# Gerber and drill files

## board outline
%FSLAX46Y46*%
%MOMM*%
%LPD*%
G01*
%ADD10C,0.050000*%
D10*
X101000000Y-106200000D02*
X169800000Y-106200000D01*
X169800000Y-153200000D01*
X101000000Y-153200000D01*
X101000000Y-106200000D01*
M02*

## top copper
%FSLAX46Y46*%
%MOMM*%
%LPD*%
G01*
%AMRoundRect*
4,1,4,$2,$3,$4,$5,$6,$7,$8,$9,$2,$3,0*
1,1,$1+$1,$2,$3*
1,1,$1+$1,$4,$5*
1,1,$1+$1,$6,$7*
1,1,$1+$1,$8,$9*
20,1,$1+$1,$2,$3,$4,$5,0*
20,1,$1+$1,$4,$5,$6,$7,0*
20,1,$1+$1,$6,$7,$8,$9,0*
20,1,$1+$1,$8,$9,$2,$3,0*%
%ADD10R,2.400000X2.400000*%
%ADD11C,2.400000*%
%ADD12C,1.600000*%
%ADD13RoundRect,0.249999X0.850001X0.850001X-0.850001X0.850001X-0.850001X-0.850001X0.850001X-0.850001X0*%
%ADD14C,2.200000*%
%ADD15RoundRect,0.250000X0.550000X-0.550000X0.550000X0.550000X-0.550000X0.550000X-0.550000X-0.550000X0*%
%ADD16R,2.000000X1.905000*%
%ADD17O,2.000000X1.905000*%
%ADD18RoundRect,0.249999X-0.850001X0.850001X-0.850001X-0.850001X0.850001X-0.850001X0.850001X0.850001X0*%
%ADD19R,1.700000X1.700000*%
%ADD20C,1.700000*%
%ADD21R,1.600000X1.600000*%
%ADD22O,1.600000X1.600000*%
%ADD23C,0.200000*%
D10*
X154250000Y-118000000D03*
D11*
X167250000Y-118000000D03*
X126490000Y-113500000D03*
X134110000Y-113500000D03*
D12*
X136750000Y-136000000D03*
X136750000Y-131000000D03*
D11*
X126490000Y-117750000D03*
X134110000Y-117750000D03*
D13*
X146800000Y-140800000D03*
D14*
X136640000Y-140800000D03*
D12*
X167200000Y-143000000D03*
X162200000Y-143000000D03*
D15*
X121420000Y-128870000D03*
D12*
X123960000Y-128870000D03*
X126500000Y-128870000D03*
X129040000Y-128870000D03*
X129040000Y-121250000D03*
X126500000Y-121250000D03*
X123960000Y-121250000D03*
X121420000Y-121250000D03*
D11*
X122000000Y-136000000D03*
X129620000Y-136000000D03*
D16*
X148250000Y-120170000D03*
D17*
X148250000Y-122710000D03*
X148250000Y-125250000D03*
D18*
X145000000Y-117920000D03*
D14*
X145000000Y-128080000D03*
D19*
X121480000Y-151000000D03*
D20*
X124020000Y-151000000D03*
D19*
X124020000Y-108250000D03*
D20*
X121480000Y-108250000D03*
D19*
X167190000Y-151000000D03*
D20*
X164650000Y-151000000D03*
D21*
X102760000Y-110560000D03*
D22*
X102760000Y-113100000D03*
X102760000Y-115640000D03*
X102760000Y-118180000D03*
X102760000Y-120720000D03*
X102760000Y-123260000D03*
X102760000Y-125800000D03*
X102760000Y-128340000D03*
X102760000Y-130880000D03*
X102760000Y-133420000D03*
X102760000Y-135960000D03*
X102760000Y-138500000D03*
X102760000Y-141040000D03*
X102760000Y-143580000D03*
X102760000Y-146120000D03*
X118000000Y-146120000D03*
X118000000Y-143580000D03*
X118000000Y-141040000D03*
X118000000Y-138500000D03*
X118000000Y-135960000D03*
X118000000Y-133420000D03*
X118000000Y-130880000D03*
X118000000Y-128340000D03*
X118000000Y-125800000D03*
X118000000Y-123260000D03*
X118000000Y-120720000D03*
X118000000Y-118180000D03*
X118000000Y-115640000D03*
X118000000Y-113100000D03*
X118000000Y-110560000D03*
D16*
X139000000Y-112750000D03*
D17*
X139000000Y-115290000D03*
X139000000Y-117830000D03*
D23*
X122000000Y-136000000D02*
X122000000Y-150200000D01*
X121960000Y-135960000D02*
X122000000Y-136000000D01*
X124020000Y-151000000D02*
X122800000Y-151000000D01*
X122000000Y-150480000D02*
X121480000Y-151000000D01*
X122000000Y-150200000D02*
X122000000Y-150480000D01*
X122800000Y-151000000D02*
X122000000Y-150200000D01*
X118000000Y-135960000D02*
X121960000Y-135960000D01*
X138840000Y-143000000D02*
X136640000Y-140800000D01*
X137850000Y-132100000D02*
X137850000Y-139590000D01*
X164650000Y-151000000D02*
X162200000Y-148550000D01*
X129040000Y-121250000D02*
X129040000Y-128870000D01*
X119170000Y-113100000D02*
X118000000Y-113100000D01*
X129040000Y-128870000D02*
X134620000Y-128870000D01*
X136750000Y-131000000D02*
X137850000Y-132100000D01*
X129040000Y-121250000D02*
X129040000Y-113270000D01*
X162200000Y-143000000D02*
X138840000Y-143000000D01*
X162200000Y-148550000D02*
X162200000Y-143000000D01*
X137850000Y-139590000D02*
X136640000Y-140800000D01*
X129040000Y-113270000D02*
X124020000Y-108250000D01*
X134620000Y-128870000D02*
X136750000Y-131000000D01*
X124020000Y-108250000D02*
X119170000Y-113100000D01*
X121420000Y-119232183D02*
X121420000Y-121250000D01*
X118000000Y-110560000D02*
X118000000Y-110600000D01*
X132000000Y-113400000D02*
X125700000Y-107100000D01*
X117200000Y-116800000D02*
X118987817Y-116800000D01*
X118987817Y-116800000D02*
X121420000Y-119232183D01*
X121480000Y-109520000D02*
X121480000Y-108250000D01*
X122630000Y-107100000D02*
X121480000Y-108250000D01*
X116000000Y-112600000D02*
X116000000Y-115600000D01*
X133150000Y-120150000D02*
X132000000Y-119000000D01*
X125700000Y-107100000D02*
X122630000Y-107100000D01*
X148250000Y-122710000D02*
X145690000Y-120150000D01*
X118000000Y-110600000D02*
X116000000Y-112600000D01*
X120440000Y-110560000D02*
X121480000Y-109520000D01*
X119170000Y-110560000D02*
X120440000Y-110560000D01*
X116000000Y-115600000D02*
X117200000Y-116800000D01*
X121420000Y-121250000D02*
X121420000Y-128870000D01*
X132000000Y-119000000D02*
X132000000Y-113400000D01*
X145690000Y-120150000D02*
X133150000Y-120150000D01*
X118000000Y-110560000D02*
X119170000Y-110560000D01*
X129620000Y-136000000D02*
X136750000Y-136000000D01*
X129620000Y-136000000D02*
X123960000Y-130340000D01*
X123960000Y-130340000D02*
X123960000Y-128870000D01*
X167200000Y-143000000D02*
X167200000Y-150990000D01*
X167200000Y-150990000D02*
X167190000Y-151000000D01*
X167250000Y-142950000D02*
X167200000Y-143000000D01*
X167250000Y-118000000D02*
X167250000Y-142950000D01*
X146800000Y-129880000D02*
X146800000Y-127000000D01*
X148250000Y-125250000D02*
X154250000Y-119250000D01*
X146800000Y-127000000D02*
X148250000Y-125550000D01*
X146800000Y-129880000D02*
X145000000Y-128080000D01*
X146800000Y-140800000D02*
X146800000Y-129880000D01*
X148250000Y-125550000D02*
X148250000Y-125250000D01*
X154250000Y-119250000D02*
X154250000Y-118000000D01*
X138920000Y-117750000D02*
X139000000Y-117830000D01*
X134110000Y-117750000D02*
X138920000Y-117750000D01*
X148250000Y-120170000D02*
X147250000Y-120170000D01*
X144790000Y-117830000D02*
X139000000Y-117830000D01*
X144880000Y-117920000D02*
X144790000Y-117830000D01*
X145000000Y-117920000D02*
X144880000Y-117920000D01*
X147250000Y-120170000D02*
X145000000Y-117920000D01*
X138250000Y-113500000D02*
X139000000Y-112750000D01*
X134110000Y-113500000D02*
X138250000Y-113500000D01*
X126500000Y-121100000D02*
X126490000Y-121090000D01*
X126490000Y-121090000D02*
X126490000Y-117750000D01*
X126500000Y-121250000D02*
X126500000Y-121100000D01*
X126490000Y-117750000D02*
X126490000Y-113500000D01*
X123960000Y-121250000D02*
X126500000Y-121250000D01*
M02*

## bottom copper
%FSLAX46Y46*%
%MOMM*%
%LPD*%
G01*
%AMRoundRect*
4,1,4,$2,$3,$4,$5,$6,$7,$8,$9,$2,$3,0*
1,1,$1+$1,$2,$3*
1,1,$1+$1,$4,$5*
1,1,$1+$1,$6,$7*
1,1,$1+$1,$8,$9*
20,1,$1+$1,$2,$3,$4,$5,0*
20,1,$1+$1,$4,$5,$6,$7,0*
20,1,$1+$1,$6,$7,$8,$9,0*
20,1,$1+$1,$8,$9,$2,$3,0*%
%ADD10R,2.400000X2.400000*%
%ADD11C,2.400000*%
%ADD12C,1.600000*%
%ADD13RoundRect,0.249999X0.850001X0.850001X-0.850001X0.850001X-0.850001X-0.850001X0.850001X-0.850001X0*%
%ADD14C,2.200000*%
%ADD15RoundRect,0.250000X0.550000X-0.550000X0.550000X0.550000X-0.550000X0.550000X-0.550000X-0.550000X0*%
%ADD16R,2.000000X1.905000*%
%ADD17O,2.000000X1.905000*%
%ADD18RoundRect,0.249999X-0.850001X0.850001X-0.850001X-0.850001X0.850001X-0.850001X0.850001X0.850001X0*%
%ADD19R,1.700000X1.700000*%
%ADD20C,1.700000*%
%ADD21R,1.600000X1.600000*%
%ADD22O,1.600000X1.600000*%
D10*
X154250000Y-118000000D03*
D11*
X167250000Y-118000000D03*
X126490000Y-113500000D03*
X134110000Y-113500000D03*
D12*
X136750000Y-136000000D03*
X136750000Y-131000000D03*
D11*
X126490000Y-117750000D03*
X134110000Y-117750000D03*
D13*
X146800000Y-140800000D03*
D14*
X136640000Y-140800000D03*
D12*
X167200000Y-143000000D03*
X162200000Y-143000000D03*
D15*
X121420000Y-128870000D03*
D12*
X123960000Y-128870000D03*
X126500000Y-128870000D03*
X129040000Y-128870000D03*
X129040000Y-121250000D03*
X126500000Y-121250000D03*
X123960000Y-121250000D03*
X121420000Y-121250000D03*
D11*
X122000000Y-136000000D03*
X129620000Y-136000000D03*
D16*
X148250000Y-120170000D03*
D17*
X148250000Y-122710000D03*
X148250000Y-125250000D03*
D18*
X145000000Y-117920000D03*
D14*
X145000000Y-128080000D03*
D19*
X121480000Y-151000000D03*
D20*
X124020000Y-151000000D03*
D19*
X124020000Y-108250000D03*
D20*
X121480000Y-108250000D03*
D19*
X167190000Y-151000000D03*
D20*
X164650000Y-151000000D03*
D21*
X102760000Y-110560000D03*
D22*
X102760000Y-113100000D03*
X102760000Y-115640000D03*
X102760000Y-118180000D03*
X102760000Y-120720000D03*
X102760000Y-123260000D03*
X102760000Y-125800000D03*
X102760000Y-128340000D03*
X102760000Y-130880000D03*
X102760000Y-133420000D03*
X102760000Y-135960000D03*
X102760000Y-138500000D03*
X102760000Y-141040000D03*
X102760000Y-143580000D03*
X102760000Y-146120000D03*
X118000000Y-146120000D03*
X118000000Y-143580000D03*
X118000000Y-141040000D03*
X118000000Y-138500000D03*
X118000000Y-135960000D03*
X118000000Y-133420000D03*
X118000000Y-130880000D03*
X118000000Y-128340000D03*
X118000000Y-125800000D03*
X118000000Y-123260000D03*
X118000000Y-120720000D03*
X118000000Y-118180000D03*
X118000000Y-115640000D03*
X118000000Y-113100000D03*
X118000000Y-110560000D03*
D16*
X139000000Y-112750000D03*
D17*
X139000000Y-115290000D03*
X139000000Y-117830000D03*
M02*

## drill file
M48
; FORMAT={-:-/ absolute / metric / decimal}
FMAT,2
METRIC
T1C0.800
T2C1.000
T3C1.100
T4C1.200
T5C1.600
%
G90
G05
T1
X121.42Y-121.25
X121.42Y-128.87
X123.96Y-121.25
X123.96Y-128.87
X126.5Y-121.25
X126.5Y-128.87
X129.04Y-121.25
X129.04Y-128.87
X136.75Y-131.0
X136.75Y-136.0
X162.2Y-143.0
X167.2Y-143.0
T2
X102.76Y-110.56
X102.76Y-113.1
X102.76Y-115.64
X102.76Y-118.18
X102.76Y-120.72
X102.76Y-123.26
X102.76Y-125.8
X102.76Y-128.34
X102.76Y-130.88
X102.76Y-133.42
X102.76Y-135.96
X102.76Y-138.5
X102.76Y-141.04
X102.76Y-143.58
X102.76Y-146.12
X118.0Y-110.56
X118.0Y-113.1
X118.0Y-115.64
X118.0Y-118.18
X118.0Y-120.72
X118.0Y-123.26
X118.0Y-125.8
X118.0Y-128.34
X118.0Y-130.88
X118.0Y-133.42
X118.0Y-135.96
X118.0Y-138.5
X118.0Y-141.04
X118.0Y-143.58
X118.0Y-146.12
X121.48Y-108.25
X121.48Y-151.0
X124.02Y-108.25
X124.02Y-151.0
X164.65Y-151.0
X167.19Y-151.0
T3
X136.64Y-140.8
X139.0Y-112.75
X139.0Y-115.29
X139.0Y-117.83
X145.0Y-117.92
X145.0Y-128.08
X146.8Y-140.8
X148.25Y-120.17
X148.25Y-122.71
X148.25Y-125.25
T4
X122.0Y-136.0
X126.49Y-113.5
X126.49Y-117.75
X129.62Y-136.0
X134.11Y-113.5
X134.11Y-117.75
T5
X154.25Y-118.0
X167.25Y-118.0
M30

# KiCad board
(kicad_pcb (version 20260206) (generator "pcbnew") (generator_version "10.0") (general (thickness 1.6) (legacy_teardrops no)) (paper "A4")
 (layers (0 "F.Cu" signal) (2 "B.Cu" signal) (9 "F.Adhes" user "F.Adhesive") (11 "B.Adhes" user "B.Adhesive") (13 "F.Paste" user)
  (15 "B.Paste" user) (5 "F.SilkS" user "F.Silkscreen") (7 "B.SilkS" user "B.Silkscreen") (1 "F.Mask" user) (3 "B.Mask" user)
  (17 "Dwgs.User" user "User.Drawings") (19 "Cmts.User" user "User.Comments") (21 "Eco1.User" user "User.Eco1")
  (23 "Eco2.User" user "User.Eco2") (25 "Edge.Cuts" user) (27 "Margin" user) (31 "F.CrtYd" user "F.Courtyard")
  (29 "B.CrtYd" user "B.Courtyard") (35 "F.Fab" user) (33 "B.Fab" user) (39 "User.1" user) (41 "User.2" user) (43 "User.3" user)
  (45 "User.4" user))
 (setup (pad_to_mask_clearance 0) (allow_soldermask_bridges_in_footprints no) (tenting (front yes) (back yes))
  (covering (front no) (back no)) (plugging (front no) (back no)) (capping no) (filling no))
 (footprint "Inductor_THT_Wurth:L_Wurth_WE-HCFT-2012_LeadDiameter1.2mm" (layer "F.Cu") (at 154.25 118)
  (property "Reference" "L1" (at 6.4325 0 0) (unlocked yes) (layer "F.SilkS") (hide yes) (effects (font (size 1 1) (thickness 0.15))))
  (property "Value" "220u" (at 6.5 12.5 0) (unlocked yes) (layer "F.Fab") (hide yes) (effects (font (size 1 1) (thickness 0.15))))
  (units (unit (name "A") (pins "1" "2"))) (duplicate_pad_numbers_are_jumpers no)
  (pad "1" thru_hole rect (at 0 0) (size 2.4 2.4) (drill 1.6) (layers "*.Cu" "*.Mask") (remove_unused_layers no) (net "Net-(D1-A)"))
  (pad "2" thru_hole circle (at 13 0) (size 2.4 2.4) (drill 1.6) (layers "*.Cu" "*.Mask") (remove_unused_layers no) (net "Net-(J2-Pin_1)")))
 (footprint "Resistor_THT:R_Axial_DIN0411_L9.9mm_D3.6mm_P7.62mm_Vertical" (layer "F.Cu") (at 126.49 113.5)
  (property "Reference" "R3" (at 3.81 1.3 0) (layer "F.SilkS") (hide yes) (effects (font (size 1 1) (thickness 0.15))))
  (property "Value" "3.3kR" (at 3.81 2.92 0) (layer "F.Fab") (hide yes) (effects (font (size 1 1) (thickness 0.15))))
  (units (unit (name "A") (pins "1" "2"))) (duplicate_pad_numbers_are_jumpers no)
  (pad "1" thru_hole circle (at 0 0) (size 2.4 2.4) (drill 1.2) (layers "*.Cu" "*.Mask") (remove_unused_layers no) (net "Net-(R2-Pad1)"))
  (pad "2" thru_hole circle (at 7.62 0) (size 2.4 2.4) (drill 1.2) (layers "*.Cu" "*.Mask") (remove_unused_layers no)
   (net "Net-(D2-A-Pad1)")))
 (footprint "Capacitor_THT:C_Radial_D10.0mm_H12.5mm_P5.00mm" (layer "F.Cu") (at 136.75 136 90)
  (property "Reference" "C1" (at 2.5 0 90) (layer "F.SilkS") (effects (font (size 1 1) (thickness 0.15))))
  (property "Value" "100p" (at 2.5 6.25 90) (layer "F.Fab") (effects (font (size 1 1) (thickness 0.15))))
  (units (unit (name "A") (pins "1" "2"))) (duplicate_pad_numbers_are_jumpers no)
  (pad "1" thru_hole circle (at 0 0 90) (size 1.6 1.6) (drill 0.8) (layers "*.Cu" "*.Mask") (remove_unused_layers no) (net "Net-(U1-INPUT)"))
  (pad "2" thru_hole circle (at 5 0 90) (size 1.6 1.6) (drill 0.8) (layers "*.Cu" "*.Mask") (remove_unused_layers no) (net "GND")))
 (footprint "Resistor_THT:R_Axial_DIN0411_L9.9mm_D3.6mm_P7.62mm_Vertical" (layer "F.Cu") (at 126.49 117.75)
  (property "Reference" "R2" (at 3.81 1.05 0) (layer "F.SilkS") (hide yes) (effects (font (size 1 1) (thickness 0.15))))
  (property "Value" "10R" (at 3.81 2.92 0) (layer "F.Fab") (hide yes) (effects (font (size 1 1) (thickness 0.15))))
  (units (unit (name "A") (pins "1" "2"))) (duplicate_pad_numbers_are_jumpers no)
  (pad "1" thru_hole circle (at 0 0) (size 2.4 2.4) (drill 1.2) (layers "*.Cu" "*.Mask") (remove_unused_layers no) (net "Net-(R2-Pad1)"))
  (pad "2" thru_hole circle (at 7.62 0) (size 2.4 2.4) (drill 1.2) (layers "*.Cu" "*.Mask") (remove_unused_layers no) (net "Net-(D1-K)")))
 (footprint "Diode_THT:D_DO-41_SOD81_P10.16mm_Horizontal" (layer "F.Cu") (at 146.8 140.8 180)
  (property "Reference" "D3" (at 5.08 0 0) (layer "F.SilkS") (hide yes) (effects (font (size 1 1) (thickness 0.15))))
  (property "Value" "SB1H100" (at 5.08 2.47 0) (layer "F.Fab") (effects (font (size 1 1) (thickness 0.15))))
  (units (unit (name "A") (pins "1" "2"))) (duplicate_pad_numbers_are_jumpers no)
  (pad "1" thru_hole roundrect (at 0 0 180) (size 2.2 2.2) (drill 1.1) (layers "*.Cu" "*.Mask") (remove_unused_layers no)
   (roundrect_rratio 0.113636) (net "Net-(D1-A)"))
  (pad "2" thru_hole circle (at 10.16 0 180) (size 2.2 2.2) (drill 1.1) (layers "*.Cu" "*.Mask") (remove_unused_layers no) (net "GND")))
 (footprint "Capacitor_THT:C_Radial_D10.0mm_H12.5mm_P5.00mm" (layer "F.Cu") (at 167.2 143 180)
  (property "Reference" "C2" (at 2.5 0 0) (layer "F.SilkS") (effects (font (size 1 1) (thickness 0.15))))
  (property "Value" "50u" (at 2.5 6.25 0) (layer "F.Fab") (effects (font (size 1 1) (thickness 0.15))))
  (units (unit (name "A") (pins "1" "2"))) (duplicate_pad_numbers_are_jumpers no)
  (pad "1" thru_hole circle (at 0 0 180) (size 1.6 1.6) (drill 0.8) (layers "*.Cu" "*.Mask") (remove_unused_layers no)
   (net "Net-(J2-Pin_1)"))
  (pad "2" thru_hole circle (at 5 0 180) (size 1.6 1.6) (drill 0.8) (layers "*.Cu" "*.Mask") (remove_unused_layers no) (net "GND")))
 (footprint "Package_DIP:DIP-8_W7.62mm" (layer "F.Cu") (at 121.42 128.87 90)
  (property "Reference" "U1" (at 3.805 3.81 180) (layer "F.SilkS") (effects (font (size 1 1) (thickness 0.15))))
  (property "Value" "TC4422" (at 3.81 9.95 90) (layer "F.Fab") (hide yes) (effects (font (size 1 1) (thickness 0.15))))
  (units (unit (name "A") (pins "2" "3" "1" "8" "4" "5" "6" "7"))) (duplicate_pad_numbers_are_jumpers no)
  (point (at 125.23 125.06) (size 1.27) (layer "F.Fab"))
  (pad "1" thru_hole roundrect (at 0 0 90) (size 1.6 1.6) (drill 0.8) (layers "*.Cu" "*.Mask") (remove_unused_layers no)
   (roundrect_rratio 0.15625) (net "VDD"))
  (pad "2" thru_hole circle (at 0 2.54 90) (size 1.6 1.6) (drill 0.8) (layers "*.Cu" "*.Mask") (remove_unused_layers no)
   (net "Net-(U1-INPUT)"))
  (pad "3" thru_hole circle (at 0 5.08 90) (size 1.6 1.6) (drill 0.8) (layers "*.Cu" "*.Mask") (remove_unused_layers no)
   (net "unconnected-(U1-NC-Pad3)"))
  (pad "4" thru_hole circle (at 0 7.62 90) (size 1.6 1.6) (drill 0.8) (layers "*.Cu" "*.Mask") (remove_unused_layers no) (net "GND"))
  (pad "5" thru_hole circle (at 7.62 7.62 90) (size 1.6 1.6) (drill 0.8) (layers "*.Cu" "*.Mask") (remove_unused_layers no) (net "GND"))
  (pad "6" thru_hole circle (at 7.62 5.08 90) (size 1.6 1.6) (drill 0.8) (layers "*.Cu" "*.Mask") (remove_unused_layers no)
   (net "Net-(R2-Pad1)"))
  (pad "7" thru_hole circle (at 7.62 2.54 90) (size 1.6 1.6) (drill 0.8) (layers "*.Cu" "*.Mask") (remove_unused_layers no)
   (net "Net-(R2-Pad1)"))
  (pad "8" thru_hole circle (at 7.62 0 90) (size 1.6 1.6) (drill 0.8) (layers "*.Cu" "*.Mask") (remove_unused_layers no) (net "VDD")))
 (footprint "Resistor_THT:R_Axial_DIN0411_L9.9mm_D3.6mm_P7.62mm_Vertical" (layer "F.Cu") (at 122 136)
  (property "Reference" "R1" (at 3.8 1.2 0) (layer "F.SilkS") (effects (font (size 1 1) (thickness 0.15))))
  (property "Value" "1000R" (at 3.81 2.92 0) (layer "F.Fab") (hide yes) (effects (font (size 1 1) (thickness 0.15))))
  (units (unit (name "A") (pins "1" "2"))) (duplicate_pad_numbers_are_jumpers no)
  (pad "1" thru_hole circle (at 0 0) (size 2.4 2.4) (drill 1.2) (layers "*.Cu" "*.Mask") (remove_unused_layers no) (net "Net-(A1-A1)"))
  (pad "2" thru_hole circle (at 7.62 0) (size 2.4 2.4) (drill 1.2) (layers "*.Cu" "*.Mask") (remove_unused_layers no) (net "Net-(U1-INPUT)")))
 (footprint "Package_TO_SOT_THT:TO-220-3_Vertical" (layer "F.Cu") (at 148.25 120.17 -90)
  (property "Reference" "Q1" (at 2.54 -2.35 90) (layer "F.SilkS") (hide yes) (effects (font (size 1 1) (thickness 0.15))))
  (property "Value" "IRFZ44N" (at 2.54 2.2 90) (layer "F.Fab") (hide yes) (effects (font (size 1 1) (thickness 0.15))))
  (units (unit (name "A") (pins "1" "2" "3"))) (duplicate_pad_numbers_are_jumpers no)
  (pad "1" thru_hole rect (at 0 0 270) (size 1.905 2) (drill 1.1) (layers "*.Cu" "*.Mask") (remove_unused_layers no) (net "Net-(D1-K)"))
  (pad "2" thru_hole oval (at 2.54 0 270) (size 1.905 2) (drill 1.1) (layers "*.Cu" "*.Mask") (remove_unused_layers no) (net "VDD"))
  (pad "3" thru_hole oval (at 5.08 0 270) (size 1.905 2) (drill 1.1) (layers "*.Cu" "*.Mask") (remove_unused_layers no) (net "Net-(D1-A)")))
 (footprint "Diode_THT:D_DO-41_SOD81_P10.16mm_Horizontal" (layer "F.Cu") (at 145 117.92 -90)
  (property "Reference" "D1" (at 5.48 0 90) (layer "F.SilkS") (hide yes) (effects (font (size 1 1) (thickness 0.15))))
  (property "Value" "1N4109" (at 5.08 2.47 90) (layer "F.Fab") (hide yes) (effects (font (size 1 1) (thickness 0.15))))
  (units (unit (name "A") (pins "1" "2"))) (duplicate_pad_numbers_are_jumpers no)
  (pad "1" thru_hole roundrect (at 0 0 270) (size 2.2 2.2) (drill 1.1) (layers "*.Cu" "*.Mask") (remove_unused_layers no)
   (roundrect_rratio 0.113636) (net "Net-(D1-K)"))
  (pad "2" thru_hole circle (at 10.16 0 270) (size 2.2 2.2) (drill 1.1) (layers "*.Cu" "*.Mask") (remove_unused_layers no)
   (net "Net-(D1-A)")))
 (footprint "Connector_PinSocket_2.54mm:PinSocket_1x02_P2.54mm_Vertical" (layer "F.Cu") (at 121.48 151 90)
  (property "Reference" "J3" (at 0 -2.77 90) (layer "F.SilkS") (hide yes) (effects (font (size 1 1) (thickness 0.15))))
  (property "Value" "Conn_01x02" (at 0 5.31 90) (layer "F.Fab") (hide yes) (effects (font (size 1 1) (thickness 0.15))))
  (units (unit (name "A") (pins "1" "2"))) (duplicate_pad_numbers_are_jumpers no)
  (pad "1" thru_hole rect (at 0 0 90) (size 1.7 1.7) (drill 1) (layers "*.Cu" "*.Mask") (remove_unused_layers no) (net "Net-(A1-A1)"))
  (pad "2" thru_hole circle (at 0 2.54 90) (size 1.7 1.7) (drill 1) (layers "*.Cu" "*.Mask") (remove_unused_layers no) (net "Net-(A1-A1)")))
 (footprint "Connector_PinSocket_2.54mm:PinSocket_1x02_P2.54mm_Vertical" (layer "F.Cu") (at 124.02 108.25 -90)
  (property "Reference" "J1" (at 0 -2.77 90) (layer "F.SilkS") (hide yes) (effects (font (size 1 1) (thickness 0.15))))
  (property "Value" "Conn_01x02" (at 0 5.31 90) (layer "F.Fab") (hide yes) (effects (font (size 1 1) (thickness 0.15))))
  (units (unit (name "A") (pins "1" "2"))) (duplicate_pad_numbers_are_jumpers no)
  (pad "1" thru_hole rect (at 0 0 270) (size 1.7 1.7) (drill 1) (layers "*.Cu" "*.Mask") (remove_unused_layers no) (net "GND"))
  (pad "2" thru_hole circle (at 0 2.54 270) (size 1.7 1.7) (drill 1) (layers "*.Cu" "*.Mask") (remove_unused_layers no) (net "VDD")))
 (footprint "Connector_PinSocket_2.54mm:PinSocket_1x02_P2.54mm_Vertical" (layer "F.Cu") (at 167.19 151 -90)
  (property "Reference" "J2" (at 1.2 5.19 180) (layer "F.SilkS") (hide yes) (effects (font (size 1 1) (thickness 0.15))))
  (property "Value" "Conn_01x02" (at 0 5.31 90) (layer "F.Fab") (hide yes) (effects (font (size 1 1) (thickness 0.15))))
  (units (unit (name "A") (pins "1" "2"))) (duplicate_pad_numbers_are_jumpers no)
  (pad "1" thru_hole rect (at 0 0 270) (size 1.7 1.7) (drill 1) (layers "*.Cu" "*.Mask") (remove_unused_layers no) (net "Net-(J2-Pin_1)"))
  (pad "2" thru_hole circle (at 0 2.54 270) (size 1.7 1.7) (drill 1) (layers "*.Cu" "*.Mask") (remove_unused_layers no) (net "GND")))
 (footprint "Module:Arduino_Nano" (layer "F.Cu") (at 102.76 110.56)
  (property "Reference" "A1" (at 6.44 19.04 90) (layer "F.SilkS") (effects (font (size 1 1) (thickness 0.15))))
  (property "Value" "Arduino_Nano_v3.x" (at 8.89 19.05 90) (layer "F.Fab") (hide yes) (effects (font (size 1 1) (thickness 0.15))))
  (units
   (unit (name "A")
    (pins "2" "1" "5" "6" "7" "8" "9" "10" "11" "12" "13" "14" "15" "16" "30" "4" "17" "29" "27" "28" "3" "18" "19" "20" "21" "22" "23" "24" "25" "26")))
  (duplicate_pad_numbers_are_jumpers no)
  (pad "1" thru_hole rect (at 0 0) (size 1.6 1.6) (drill 1) (layers "*.Cu" "*.Mask") (remove_unused_layers no)
   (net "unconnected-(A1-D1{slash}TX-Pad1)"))
  (pad "2" thru_hole oval (at 0 2.54) (size 1.6 1.6) (drill 1) (layers "*.Cu" "*.Mask") (remove_unused_layers no)
   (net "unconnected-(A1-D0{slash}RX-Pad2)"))
  (pad "3" thru_hole oval (at 0 5.08) (size 1.6 1.6) (drill 1) (layers "*.Cu" "*.Mask") (remove_unused_layers no)
   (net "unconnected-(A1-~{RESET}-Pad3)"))
  (pad "4" thru_hole oval (at 0 7.62) (size 1.6 1.6) (drill 1) (layers "*.Cu" "*.Mask") (remove_unused_layers no) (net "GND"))
  (pad "5" thru_hole oval (at 0 10.16) (size 1.6 1.6) (drill 1) (layers "*.Cu" "*.Mask") (remove_unused_layers no)
   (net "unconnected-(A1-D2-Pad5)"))
  (pad "6" thru_hole oval (at 0 12.7) (size 1.6 1.6) (drill 1) (layers "*.Cu" "*.Mask") (remove_unused_layers no)
   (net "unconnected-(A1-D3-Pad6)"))
  (pad "7" thru_hole oval (at 0 15.24) (size 1.6 1.6) (drill 1) (layers "*.Cu" "*.Mask") (remove_unused_layers no)
   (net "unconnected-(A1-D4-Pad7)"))
  (pad "8" thru_hole oval (at 0 17.78) (size 1.6 1.6) (drill 1) (layers "*.Cu" "*.Mask") (remove_unused_layers no)
   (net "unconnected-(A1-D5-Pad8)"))
  (pad "9" thru_hole oval (at 0 20.32) (size 1.6 1.6) (drill 1) (layers "*.Cu" "*.Mask") (remove_unused_layers no)
   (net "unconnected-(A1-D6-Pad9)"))
  (pad "10" thru_hole oval (at 0 22.86) (size 1.6 1.6) (drill 1) (layers "*.Cu" "*.Mask") (remove_unused_layers no)
   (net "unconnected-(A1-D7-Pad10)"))
  (pad "11" thru_hole oval (at 0 25.4) (size 1.6 1.6) (drill 1) (layers "*.Cu" "*.Mask") (remove_unused_layers no)
   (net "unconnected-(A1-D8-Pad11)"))
  (pad "12" thru_hole oval (at 0 27.94) (size 1.6 1.6) (drill 1) (layers "*.Cu" "*.Mask") (remove_unused_layers no)
   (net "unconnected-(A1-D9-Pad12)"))
  (pad "13" thru_hole oval (at 0 30.48) (size 1.6 1.6) (drill 1) (layers "*.Cu" "*.Mask") (remove_unused_layers no)
   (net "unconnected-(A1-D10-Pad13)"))
  (pad "14" thru_hole oval (at 0 33.02) (size 1.6 1.6) (drill 1) (layers "*.Cu" "*.Mask") (remove_unused_layers no)
   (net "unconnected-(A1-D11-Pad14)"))
  (pad "15" thru_hole oval (at 0 35.56) (size 1.6 1.6) (drill 1) (layers "*.Cu" "*.Mask") (remove_unused_layers no)
   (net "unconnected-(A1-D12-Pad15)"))
  (pad "16" thru_hole oval (at 15.24 35.56) (size 1.6 1.6) (drill 1) (layers "*.Cu" "*.Mask") (remove_unused_layers no)
   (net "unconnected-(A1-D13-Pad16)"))
  (pad "17" thru_hole oval (at 15.24 33.02) (size 1.6 1.6) (drill 1) (layers "*.Cu" "*.Mask") (remove_unused_layers no)
   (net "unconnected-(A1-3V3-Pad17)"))
  (pad "18" thru_hole oval (at 15.24 30.48) (size 1.6 1.6) (drill 1) (layers "*.Cu" "*.Mask") (remove_unused_layers no)
   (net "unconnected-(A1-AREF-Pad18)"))
  (pad "19" thru_hole oval (at 15.24 27.94) (size 1.6 1.6) (drill 1) (layers "*.Cu" "*.Mask") (remove_unused_layers no)
   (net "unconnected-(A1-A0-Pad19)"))
  (pad "20" thru_hole oval (at 15.24 25.4) (size 1.6 1.6) (drill 1) (layers "*.Cu" "*.Mask") (remove_unused_layers no) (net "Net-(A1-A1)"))
  (pad "21" thru_hole oval (at 15.24 22.86) (size 1.6 1.6) (drill 1) (layers "*.Cu" "*.Mask") (remove_unused_layers no)
   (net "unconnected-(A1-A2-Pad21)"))
  (pad "22" thru_hole oval (at 15.24 20.32) (size 1.6 1.6) (drill 1) (layers "*.Cu" "*.Mask") (remove_unused_layers no)
   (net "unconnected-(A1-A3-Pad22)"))
  (pad "23" thru_hole oval (at 15.24 17.78) (size 1.6 1.6) (drill 1) (layers "*.Cu" "*.Mask") (remove_unused_layers no)
   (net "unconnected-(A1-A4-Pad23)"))
  (pad "24" thru_hole oval (at 15.24 15.24) (size 1.6 1.6) (drill 1) (layers "*.Cu" "*.Mask") (remove_unused_layers no)
   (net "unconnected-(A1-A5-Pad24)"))
  (pad "25" thru_hole oval (at 15.24 12.7) (size 1.6 1.6) (drill 1) (layers "*.Cu" "*.Mask") (remove_unused_layers no)
   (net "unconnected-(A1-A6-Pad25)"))
  (pad "26" thru_hole oval (at 15.24 10.16) (size 1.6 1.6) (drill 1) (layers "*.Cu" "*.Mask") (remove_unused_layers no)
   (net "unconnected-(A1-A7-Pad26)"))
  (pad "27" thru_hole oval (at 15.24 7.62) (size 1.6 1.6) (drill 1) (layers "*.Cu" "*.Mask") (remove_unused_layers no)
   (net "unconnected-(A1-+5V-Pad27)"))
  (pad "28" thru_hole oval (at 15.24 5.08) (size 1.6 1.6) (drill 1) (layers "*.Cu" "*.Mask") (remove_unused_layers no)
   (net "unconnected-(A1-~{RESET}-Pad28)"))
  (pad "29" thru_hole oval (at 15.24 2.54) (size 1.6 1.6) (drill 1) (layers "*.Cu" "*.Mask") (remove_unused_layers no) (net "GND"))
  (pad "30" thru_hole oval (at 15.24 0) (size 1.6 1.6) (drill 1) (layers "*.Cu" "*.Mask") (remove_unused_layers no) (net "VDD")))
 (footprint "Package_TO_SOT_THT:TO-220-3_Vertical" (layer "F.Cu") (at 139 112.75 -90)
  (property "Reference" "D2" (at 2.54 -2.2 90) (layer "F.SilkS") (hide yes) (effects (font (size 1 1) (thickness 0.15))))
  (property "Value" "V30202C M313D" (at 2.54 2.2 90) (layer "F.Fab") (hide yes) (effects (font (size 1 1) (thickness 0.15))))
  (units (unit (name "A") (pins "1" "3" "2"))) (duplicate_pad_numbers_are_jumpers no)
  (pad "1" thru_hole rect (at 0 0 270) (size 1.905 2) (drill 1.1) (layers "*.Cu" "*.Mask") (remove_unused_layers no) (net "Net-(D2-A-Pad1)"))
  (pad "2" thru_hole oval (at 2.54 0 270) (size 1.905 2) (drill 1.1) (layers "*.Cu" "*.Mask") (remove_unused_layers no)
   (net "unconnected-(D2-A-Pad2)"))
  (pad "3" thru_hole oval (at 5.08 0 270) (size 1.905 2) (drill 1.1) (layers "*.Cu" "*.Mask") (remove_unused_layers no) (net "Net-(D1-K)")))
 (gr_rect (start 101 106.2) (end 169.8 153.2) (stroke (width 0.05) (type default)) (fill no) (layer "Edge.Cuts"))
 (segment (start 122 136) (end 122 150.2) (width 0.2) (layer "F.Cu") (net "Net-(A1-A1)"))
 (segment (start 121.96 135.96) (end 122 136) (width 0.2) (layer "F.Cu") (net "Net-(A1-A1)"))
 (segment (start 124.02 151) (end 122.8 151) (width 0.2) (layer "F.Cu") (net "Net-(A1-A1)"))
 (segment (start 122 150.48) (end 121.48 151) (width 0.2) (layer "F.Cu") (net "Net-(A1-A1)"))
 (segment (start 122 150.2) (end 122 150.48) (width 0.2) (layer "F.Cu") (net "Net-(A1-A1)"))
 (segment (start 122.8 151) (end 122 150.2) (width 0.2) (layer "F.Cu") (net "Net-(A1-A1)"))
 (segment (start 118 135.96) (end 121.96 135.96) (width 0.2) (layer "F.Cu") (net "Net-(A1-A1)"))
 (segment (start 138.84 143) (end 136.64 140.8) (width 0.2) (layer "F.Cu") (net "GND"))
 (segment (start 137.85 132.1) (end 137.85 139.59) (width 0.2) (layer "F.Cu") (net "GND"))
 (segment (start 164.65 151) (end 162.2 148.55) (width 0.2) (layer "F.Cu") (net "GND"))
 (segment (start 129.04 121.25) (end 129.04 128.87) (width 0.2) (layer "F.Cu") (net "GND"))
 (segment (start 119.17 113.1) (end 118 113.1) (width 0.2) (layer "F.Cu") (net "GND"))
 (segment (start 129.04 128.87) (end 134.62 128.87) (width 0.2) (layer "F.Cu") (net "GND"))
 (segment (start 136.75 131) (end 137.85 132.1) (width 0.2) (layer "F.Cu") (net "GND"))
 (segment (start 129.04 121.25) (end 129.04 113.27) (width 0.2) (layer "F.Cu") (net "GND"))
 (segment (start 162.2 143) (end 138.84 143) (width 0.2) (layer "F.Cu") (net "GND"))
 (segment (start 162.2 148.55) (end 162.2 143) (width 0.2) (layer "F.Cu") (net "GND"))
 (segment (start 137.85 139.59) (end 136.64 140.8) (width 0.2) (layer "F.Cu") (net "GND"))
 (segment (start 129.04 113.27) (end 124.02 108.25) (width 0.2) (layer "F.Cu") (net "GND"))
 (segment (start 134.62 128.87) (end 136.75 131) (width 0.2) (layer "F.Cu") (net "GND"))
 (segment (start 124.02 108.25) (end 119.17 113.1) (width 0.2) (layer "F.Cu") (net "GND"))
 (segment (start 121.42 119.232183) (end 121.42 121.25) (width 0.2) (layer "F.Cu") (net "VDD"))
 (segment (start 118 110.56) (end 118 110.6) (width 0.2) (layer "F.Cu") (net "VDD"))
 (segment (start 132 113.4) (end 125.7 107.1) (width 0.2) (layer "F.Cu") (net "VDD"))
 (segment (start 117.2 116.8) (end 118.987817 116.8) (width 0.2) (layer "F.Cu") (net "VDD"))
 (segment (start 118.987817 116.8) (end 121.42 119.232183) (width 0.2) (layer "F.Cu") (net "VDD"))
 (segment (start 121.48 109.52) (end 121.48 108.25) (width 0.2) (layer "F.Cu") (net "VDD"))
 (segment (start 122.63 107.1) (end 121.48 108.25) (width 0.2) (layer "F.Cu") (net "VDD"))
 (segment (start 116 112.6) (end 116 115.6) (width 0.2) (layer "F.Cu") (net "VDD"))
 (segment (start 133.15 120.15) (end 132 119) (width 0.2) (layer "F.Cu") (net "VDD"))
 (segment (start 125.7 107.1) (end 122.63 107.1) (width 0.2) (layer "F.Cu") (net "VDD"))
 (segment (start 148.25 122.71) (end 145.69 120.15) (width 0.2) (layer "F.Cu") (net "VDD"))
 (segment (start 118 110.6) (end 116 112.6) (width 0.2) (layer "F.Cu") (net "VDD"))
 (segment (start 120.44 110.56) (end 121.48 109.52) (width 0.2) (layer "F.Cu") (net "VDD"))
 (segment (start 119.17 110.56) (end 120.44 110.56) (width 0.2) (layer "F.Cu") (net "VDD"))
 (segment (start 116 115.6) (end 117.2 116.8) (width 0.2) (layer "F.Cu") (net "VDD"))
 (segment (start 121.42 121.25) (end 121.42 128.87) (width 0.2) (layer "F.Cu") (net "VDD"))
 (segment (start 132 119) (end 132 113.4) (width 0.2) (layer "F.Cu") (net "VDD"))
 (segment (start 145.69 120.15) (end 133.15 120.15) (width 0.2) (layer "F.Cu") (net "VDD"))
 (segment (start 118 110.56) (end 119.17 110.56) (width 0.2) (layer "F.Cu") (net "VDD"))
 (segment (start 129.62 136) (end 136.75 136) (width 0.2) (layer "F.Cu") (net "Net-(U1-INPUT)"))
 (segment (start 129.62 136) (end 123.96 130.34) (width 0.2) (layer "F.Cu") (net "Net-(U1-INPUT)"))
 (segment (start 123.96 130.34) (end 123.96 128.87) (width 0.2) (layer "F.Cu") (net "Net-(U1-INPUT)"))
 (segment (start 167.2 143) (end 167.2 150.99) (width 0.2) (layer "F.Cu") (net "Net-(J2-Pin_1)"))
 (segment (start 167.2 150.99) (end 167.19 151) (width 0.2) (layer "F.Cu") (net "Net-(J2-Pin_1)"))
 (segment (start 167.25 142.95) (end 167.2 143) (width 0.2) (layer "F.Cu") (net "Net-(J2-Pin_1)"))
 (segment (start 167.25 118) (end 167.25 142.95) (width 0.2) (layer "F.Cu") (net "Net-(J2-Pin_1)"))
 (segment (start 146.8 129.88) (end 146.8 127) (width 0.2) (layer "F.Cu") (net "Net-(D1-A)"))
 (segment (start 148.25 125.25) (end 154.25 119.25) (width 0.2) (layer "F.Cu") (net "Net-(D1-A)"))
 (segment (start 146.8 127) (end 148.25 125.55) (width 0.2) (layer "F.Cu") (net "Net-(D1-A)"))
 (segment (start 146.8 129.88) (end 145 128.08) (width 0.2) (layer "F.Cu") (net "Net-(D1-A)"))
 (segment (start 146.8 140.8) (end 146.8 129.88) (width 0.2) (layer "F.Cu") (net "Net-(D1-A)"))
 (segment (start 148.25 125.55) (end 148.25 125.25) (width 0.2) (layer "F.Cu") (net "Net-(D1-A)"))
 (segment (start 154.25 119.25) (end 154.25 118) (width 0.2) (layer "F.Cu") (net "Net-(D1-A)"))
 (segment (start 138.92 117.75) (end 139 117.83) (width 0.2) (layer "F.Cu") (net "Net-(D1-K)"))
 (segment (start 134.11 117.75) (end 138.92 117.75) (width 0.2) (layer "F.Cu") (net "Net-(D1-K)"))
 (segment (start 148.25 120.17) (end 147.25 120.17) (width 0.2) (layer "F.Cu") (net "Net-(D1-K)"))
 (segment (start 144.79 117.83) (end 139 117.83) (width 0.2) (layer "F.Cu") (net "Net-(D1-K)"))
 (segment (start 144.88 117.92) (end 144.79 117.83) (width 0.2) (layer "F.Cu") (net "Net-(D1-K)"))
 (segment (start 145 117.92) (end 144.88 117.92) (width 0.2) (layer "F.Cu") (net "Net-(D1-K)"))
 (segment (start 147.25 120.17) (end 145 117.92) (width 0.2) (layer "F.Cu") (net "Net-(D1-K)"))
 (segment (start 138.25 113.5) (end 139 112.75) (width 0.2) (layer "F.Cu") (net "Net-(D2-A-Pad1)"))
 (segment (start 134.11 113.5) (end 138.25 113.5) (width 0.2) (layer "F.Cu") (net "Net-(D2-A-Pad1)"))
 (segment (start 126.5 121.1) (end 126.49 121.09) (width 0.2) (layer "F.Cu") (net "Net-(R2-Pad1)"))
 (segment (start 126.49 121.09) (end 126.49 117.75) (width 0.2) (layer "F.Cu") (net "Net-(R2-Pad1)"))
 (segment (start 126.5 121.25) (end 126.5 121.1) (width 0.2) (layer "F.Cu") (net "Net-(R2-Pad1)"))
 (segment (start 126.49 117.75) (end 126.49 113.5) (width 0.2) (layer "F.Cu") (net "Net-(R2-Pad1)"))
 (segment (start 123.96 121.25) (end 126.5 121.25) (width 0.2) (layer "F.Cu") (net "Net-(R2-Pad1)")))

